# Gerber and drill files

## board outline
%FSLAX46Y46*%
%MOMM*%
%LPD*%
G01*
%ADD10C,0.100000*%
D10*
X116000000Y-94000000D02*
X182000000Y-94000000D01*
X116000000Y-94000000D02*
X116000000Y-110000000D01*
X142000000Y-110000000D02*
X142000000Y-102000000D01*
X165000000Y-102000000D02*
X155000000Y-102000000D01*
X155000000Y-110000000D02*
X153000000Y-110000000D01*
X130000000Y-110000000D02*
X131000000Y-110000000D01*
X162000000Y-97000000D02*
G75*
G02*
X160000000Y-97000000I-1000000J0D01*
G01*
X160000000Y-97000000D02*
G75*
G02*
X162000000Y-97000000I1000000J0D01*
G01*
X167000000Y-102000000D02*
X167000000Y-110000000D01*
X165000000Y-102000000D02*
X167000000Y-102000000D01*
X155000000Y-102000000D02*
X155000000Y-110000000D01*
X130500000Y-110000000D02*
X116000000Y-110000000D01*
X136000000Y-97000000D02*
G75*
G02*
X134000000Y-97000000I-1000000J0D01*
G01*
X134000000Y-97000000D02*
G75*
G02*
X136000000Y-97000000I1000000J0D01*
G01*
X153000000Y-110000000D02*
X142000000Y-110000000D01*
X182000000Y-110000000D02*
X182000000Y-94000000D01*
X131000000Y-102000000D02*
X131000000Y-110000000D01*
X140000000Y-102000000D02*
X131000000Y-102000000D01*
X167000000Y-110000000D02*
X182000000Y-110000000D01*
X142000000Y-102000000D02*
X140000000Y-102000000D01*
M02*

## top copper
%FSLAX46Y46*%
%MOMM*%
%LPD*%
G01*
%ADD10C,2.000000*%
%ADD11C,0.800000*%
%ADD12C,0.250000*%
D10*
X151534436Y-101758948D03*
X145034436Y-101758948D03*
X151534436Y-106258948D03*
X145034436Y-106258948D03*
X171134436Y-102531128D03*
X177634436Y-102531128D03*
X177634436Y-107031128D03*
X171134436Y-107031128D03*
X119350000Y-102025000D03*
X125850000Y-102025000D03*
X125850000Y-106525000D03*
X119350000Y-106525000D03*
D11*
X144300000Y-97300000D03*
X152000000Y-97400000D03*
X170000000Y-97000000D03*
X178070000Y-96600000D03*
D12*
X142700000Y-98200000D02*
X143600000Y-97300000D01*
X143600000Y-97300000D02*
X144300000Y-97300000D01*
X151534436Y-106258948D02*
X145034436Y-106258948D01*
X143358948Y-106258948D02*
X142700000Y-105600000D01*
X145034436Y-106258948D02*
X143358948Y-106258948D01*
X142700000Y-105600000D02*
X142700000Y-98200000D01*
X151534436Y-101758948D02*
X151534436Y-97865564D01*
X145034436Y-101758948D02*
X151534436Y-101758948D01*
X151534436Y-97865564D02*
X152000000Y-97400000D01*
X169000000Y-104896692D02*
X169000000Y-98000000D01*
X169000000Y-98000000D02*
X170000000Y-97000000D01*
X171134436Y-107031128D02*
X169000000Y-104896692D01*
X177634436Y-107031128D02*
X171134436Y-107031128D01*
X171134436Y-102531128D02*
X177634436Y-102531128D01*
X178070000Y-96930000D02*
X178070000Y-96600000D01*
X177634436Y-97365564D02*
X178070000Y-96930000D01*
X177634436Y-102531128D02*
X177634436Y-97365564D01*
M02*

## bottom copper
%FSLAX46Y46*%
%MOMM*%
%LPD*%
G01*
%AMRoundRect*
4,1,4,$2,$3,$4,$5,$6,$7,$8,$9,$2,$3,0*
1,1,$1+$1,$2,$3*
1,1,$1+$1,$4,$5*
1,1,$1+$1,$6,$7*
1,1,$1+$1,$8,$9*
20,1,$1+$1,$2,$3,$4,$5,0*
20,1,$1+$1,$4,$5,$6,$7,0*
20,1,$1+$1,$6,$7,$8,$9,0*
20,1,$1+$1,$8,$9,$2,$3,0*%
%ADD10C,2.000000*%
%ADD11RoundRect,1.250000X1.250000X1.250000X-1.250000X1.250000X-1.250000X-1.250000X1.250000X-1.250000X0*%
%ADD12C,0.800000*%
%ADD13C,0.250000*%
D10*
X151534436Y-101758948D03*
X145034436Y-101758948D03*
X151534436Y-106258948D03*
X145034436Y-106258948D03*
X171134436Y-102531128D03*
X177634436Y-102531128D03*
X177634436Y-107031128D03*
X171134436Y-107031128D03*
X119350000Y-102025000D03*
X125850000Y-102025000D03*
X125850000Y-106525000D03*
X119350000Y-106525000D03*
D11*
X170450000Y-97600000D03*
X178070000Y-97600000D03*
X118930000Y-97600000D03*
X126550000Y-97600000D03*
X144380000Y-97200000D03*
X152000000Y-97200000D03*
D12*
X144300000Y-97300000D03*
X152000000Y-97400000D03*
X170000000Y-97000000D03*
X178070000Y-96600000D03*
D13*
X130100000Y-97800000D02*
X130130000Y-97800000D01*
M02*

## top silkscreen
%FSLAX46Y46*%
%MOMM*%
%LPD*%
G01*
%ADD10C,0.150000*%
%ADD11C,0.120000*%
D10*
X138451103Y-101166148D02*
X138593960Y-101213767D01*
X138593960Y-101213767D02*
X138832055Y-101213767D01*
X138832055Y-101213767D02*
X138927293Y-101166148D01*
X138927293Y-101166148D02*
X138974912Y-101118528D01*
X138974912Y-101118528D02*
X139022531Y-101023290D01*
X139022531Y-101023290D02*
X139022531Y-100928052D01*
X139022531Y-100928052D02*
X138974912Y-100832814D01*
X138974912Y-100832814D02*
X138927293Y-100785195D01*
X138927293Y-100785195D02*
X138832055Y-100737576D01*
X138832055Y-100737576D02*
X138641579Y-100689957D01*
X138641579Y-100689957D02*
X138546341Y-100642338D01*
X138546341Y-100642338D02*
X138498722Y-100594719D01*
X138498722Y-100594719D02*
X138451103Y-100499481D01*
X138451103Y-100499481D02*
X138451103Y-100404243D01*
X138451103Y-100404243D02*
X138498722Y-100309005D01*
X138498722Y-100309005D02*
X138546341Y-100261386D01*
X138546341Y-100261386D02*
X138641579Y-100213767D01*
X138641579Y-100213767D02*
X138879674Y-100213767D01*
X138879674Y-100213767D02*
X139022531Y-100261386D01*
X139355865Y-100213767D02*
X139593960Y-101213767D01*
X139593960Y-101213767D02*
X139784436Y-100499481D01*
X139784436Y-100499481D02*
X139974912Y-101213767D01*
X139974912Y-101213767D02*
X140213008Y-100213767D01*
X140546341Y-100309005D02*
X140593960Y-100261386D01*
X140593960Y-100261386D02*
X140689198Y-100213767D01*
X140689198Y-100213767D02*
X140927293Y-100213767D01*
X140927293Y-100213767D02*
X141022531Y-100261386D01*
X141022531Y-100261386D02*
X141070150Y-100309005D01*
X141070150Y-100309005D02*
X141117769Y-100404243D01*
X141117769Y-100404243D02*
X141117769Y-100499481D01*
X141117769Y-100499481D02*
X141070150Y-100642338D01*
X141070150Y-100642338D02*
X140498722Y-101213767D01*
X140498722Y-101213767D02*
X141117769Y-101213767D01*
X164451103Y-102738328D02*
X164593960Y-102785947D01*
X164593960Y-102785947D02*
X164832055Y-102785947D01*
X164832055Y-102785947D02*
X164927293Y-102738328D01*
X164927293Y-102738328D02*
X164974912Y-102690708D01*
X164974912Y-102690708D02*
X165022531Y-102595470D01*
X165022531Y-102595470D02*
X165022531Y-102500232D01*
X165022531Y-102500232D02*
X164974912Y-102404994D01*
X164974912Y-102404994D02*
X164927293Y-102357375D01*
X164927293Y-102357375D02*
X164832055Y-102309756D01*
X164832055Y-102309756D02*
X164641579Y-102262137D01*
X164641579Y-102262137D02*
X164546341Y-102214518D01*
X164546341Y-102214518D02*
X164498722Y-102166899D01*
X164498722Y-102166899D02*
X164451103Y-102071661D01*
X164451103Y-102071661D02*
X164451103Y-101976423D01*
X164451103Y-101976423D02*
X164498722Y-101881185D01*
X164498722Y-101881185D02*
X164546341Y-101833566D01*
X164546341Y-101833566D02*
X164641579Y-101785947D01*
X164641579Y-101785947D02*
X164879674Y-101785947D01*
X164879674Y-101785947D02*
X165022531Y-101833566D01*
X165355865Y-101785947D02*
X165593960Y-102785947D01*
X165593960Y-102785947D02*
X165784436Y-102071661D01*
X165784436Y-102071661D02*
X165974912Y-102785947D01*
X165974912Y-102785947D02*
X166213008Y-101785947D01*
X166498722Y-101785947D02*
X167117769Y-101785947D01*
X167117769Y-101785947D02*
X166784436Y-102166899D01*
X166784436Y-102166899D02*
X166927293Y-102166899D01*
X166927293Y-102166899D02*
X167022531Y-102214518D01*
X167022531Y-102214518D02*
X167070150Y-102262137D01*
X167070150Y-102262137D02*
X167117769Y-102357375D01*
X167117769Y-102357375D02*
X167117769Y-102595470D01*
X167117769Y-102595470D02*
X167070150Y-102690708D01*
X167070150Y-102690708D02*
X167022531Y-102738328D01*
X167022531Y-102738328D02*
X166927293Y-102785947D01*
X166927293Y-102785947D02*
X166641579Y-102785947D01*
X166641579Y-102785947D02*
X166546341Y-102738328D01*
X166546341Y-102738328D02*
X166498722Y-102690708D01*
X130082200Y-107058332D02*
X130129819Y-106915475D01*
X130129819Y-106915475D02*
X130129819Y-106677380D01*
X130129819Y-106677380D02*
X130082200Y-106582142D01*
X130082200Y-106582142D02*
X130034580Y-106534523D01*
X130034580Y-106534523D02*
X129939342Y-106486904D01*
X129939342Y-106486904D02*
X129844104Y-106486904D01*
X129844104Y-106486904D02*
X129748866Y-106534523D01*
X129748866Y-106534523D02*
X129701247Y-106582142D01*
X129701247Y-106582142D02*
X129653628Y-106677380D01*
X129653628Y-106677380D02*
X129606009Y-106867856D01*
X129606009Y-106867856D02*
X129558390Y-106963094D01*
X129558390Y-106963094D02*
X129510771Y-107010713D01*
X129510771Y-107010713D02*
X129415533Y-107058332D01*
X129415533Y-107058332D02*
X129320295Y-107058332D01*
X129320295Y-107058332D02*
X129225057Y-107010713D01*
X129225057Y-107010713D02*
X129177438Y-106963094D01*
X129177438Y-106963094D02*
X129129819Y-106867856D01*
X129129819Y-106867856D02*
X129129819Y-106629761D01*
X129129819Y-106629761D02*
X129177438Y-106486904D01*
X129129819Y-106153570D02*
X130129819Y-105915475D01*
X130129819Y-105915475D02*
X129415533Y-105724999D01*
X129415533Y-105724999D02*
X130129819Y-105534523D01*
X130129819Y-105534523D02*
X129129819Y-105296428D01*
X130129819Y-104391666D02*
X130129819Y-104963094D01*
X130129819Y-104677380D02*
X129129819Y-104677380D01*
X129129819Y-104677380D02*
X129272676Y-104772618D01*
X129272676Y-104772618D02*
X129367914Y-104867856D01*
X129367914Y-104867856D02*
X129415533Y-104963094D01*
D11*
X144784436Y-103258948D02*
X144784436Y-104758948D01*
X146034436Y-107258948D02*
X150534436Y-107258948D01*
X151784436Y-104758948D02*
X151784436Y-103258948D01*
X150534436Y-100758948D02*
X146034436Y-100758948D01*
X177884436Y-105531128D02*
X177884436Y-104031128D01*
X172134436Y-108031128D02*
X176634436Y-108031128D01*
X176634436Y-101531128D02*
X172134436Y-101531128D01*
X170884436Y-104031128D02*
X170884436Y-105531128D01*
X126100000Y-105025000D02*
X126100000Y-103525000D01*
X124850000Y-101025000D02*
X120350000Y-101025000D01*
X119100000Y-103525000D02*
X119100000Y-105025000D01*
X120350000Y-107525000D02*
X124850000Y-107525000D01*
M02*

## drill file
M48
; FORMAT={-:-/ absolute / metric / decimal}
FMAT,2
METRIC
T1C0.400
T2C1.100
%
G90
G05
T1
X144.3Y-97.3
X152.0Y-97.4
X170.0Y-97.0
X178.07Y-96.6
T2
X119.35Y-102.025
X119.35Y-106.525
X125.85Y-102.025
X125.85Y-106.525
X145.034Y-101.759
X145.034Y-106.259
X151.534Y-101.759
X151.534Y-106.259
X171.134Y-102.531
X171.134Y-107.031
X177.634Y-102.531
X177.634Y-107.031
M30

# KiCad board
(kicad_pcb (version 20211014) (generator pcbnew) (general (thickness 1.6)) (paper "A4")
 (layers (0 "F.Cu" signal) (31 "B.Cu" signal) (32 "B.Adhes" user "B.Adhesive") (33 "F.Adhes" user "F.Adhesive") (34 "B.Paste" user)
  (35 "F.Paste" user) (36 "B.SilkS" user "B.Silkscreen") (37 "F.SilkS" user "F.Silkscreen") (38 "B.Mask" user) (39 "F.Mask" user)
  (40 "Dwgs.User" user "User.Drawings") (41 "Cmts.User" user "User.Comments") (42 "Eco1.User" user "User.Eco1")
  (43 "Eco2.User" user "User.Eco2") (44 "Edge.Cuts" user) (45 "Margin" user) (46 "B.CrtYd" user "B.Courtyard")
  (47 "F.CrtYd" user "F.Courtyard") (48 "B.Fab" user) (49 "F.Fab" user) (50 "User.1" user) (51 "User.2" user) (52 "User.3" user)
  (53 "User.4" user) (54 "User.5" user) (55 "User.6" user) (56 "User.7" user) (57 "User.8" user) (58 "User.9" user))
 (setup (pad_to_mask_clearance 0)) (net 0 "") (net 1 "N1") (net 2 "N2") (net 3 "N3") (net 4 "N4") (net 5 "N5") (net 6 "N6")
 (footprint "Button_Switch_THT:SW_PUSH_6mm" (layer "F.Cu") (at 145.034436 101.758948)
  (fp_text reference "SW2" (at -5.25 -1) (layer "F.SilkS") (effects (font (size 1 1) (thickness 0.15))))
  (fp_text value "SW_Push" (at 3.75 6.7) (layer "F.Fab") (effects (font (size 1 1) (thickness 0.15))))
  (fp_line (start -0.25 1.5) (end -0.25 3) (layer "F.SilkS") (width 0.12))
  (fp_line (start 1 5.5) (end 5.5 5.5) (layer "F.SilkS") (width 0.12))
  (fp_line (start 6.75 3) (end 6.75 1.5) (layer "F.SilkS") (width 0.12))
  (fp_line (start 5.5 -1) (end 1 -1) (layer "F.SilkS") (width 0.12))
  (pad "1" thru_hole circle (at 6.5 0 90) (size 2 2) (drill 1.1) (layers *.Cu *.Mask) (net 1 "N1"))
  (pad "1" thru_hole circle (at 0 0 90) (size 2 2) (drill 1.1) (layers *.Cu *.Mask) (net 1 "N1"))
  (pad "2" thru_hole circle (at 6.5 4.5 90) (size 2 2) (drill 1.1) (layers *.Cu *.Mask) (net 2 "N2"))
  (pad "2" thru_hole circle (at 0 4.5 90) (size 2 2) (drill 1.1) (layers *.Cu *.Mask) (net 2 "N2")))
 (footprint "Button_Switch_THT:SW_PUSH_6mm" (layer "F.Cu") (at 171.134436 102.531128)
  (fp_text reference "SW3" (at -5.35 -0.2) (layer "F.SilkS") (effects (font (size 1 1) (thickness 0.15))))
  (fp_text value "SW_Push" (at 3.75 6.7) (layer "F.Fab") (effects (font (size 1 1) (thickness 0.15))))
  (fp_line (start 6.75 3) (end 6.75 1.5) (layer "F.SilkS") (width 0.12))
  (fp_line (start 1 5.5) (end 5.5 5.5) (layer "F.SilkS") (width 0.12))
  (fp_line (start 5.5 -1) (end 1 -1) (layer "F.SilkS") (width 0.12))
  (fp_line (start -0.25 1.5) (end -0.25 3) (layer "F.SilkS") (width 0.12))
  (pad "1" thru_hole circle (at 0 0 90) (size 2 2) (drill 1.1) (layers *.Cu *.Mask) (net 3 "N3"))
  (pad "1" thru_hole circle (at 6.5 0 90) (size 2 2) (drill 1.1) (layers *.Cu *.Mask) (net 3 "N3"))
  (pad "2" thru_hole circle (at 6.5 4.5 90) (size 2 2) (drill 1.1) (layers *.Cu *.Mask) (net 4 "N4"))
  (pad "2" thru_hole circle (at 0 4.5 90) (size 2 2) (drill 1.1) (layers *.Cu *.Mask) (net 4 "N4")))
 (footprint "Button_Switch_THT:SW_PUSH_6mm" (layer "F.Cu") (at 119.35 102.025)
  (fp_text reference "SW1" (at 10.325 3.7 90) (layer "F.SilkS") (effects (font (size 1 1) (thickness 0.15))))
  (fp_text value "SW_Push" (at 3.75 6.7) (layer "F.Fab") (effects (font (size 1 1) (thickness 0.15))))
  (fp_line (start 6.75 3) (end 6.75 1.5) (layer "F.SilkS") (width 0.12))
  (fp_line (start 5.5 -1) (end 1 -1) (layer "F.SilkS") (width 0.12))
  (fp_line (start -0.25 1.5) (end -0.25 3) (layer "F.SilkS") (width 0.12))
  (fp_line (start 1 5.5) (end 5.5 5.5) (layer "F.SilkS") (width 0.12))
  (pad "1" thru_hole circle (at 0 0 90) (size 2 2) (drill 1.1) (layers *.Cu *.Mask) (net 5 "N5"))
  (pad "1" thru_hole circle (at 6.5 0 90) (size 2 2) (drill 1.1) (layers *.Cu *.Mask) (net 5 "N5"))
  (pad "2" thru_hole circle (at 6.5 4.5 90) (size 2 2) (drill 1.1) (layers *.Cu *.Mask) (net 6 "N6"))
  (pad "2" thru_hole circle (at 0 4.5 90) (size 2 2) (drill 1.1) (layers *.Cu *.Mask) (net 6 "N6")))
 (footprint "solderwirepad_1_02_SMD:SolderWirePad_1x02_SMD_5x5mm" (layer "B.Cu") (at 178.07 97.6 180)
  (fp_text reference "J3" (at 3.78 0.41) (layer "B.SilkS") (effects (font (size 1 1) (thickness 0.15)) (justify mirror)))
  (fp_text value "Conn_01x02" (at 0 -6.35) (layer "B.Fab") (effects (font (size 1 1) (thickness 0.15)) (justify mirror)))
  (pad "1" smd roundrect (at 7.62 0 180) (size 5 5) (layers "B.Cu" "B.Paste" "B.Mask") (roundrect_rratio 0.25) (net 4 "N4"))
  (pad "2" smd roundrect (at 0 0 180) (size 5 5) (layers "B.Cu" "B.Paste" "B.Mask") (roundrect_rratio 0.25) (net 3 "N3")))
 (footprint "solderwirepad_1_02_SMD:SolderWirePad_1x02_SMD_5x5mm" (layer "B.Cu") (at 126.55 97.6 180)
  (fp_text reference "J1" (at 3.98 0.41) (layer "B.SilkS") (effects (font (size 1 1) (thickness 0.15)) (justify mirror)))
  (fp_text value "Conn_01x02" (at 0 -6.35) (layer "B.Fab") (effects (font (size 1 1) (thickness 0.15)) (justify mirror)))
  (pad "1" smd roundrect (at 7.62 0 180) (size 5 5) (layers "B.Cu" "B.Paste" "B.Mask") (roundrect_rratio 0.25) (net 6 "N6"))
  (pad "2" smd roundrect (at 0 0 180) (size 5 5) (layers "B.Cu" "B.Paste" "B.Mask") (roundrect_rratio 0.25) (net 5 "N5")))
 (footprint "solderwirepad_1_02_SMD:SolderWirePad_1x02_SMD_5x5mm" (layer "B.Cu") (at 152 97.2 180)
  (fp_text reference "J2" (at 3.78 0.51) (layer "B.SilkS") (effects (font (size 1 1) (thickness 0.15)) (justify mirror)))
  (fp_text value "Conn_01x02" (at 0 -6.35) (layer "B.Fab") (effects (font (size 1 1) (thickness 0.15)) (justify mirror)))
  (pad "1" smd roundrect (at 7.62 0 180) (size 5 5) (layers "B.Cu" "B.Paste" "B.Mask") (roundrect_rratio 0.25) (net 2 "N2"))
  (pad "2" smd roundrect (at 0 0 180) (size 5 5) (layers "B.Cu" "B.Paste" "B.Mask") (roundrect_rratio 0.25) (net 1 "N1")))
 (gr_line (start 116 94) (end 182 94) (layer "Edge.Cuts") (width 0.1))
 (gr_line (start 116 94) (end 116 110) (layer "Edge.Cuts") (width 0.1))
 (gr_line (start 142 110) (end 142 102) (layer "Edge.Cuts") (width 0.1))
 (gr_line (start 165 102) (end 155 102) (layer "Edge.Cuts") (width 0.1))
 (gr_line (start 155 110) (end 153 110) (layer "Edge.Cuts") (width 0.1))
 (gr_line (start 130 110) (end 131 110) (layer "Edge.Cuts") (width 0.1))
 (gr_circle (center 161 97) (end 162 97) (layer "Edge.Cuts") (width 0.1) (fill none))
 (gr_line (start 167 102) (end 167 110) (layer "Edge.Cuts") (width 0.1))
 (gr_line (start 165 102) (end 167 102) (layer "Edge.Cuts") (width 0.1))
 (gr_line (start 155 102) (end 155 110) (layer "Edge.Cuts") (width 0.1))
 (gr_line (start 130.5 110) (end 116 110) (layer "Edge.Cuts") (width 0.1))
 (gr_circle (center 135 97) (end 136 97) (layer "Edge.Cuts") (width 0.1) (fill none))
 (gr_line (start 153 110) (end 142 110) (layer "Edge.Cuts") (width 0.1))
 (gr_line (start 182 110) (end 182 94) (layer "Edge.Cuts") (width 0.1))
 (gr_line (start 131 102) (end 131 110) (layer "Edge.Cuts") (width 0.1))
 (gr_line (start 140 102) (end 131 102) (layer "Edge.Cuts") (width 0.1))
 (gr_line (start 167 110) (end 182 110) (layer "Edge.Cuts") (width 0.1))
 (gr_line (start 142 102) (end 140 102) (layer "Edge.Cuts") (width 0.1))
 (segment (start 130.1 97.8) (end 130.13 97.8) (width 0.25) (layer "B.Cu") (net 6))
 (segment (start 142.7 98.2) (end 143.6 97.3) (width 0.25) (layer "F.Cu") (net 2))
 (segment (start 143.6 97.3) (end 144.3 97.3) (width 0.25) (layer "F.Cu") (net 2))
 (segment (start 151.534436 106.258948) (end 145.034436 106.258948) (width 0.25) (layer "F.Cu") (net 2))
 (segment (start 143.358948 106.258948) (end 142.7 105.6) (width 0.25) (layer "F.Cu") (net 2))
 (segment (start 145.034436 106.258948) (end 143.358948 106.258948) (width 0.25) (layer "F.Cu") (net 2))
 (segment (start 142.7 105.6) (end 142.7 98.2) (width 0.25) (layer "F.Cu") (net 2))
 (via (at 144.3 97.3) (size 0.8) (drill 0.4) (layers "F.Cu" "B.Cu") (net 2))
 (segment (start 151.534436 101.758948) (end 151.534436 97.865564) (width 0.25) (layer "F.Cu") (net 1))
 (segment (start 145.034436 101.758948) (end 151.534436 101.758948) (width 0.25) (layer "F.Cu") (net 1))
 (segment (start 151.534436 97.865564) (end 152 97.4) (width 0.25) (layer "F.Cu") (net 1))
 (via (at 152 97.4) (size 0.8) (drill 0.4) (layers "F.Cu" "B.Cu") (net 1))
 (segment (start 169 104.896692) (end 169 98) (width 0.25) (layer "F.Cu") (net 4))
 (segment (start 169 98) (end 170 97) (width 0.25) (layer "F.Cu") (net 4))
 (segment (start 171.134436 107.031128) (end 169 104.896692) (width 0.25) (layer "F.Cu") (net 4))
 (segment (start 177.634436 107.031128) (end 171.134436 107.031128) (width 0.25) (layer "F.Cu") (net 4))
 (via (at 170 97) (size 0.8) (drill 0.4) (layers "F.Cu" "B.Cu") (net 4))
 (segment (start 171.134436 102.531128) (end 177.634436 102.531128) (width 0.25) (layer "F.Cu") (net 3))
 (segment (start 178.07 96.93) (end 178.07 96.6) (width 0.25) (layer "F.Cu") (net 3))
 (segment (start 177.634436 97.365564) (end 178.07 96.93) (width 0.25) (layer "F.Cu") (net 3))
 (segment (start 177.634436 102.531128) (end 177.634436 97.365564) (width 0.25) (layer "F.Cu") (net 3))
 (via (at 178.07 96.6) (size 0.8) (drill 0.4) (layers "F.Cu" "B.Cu") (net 3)))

